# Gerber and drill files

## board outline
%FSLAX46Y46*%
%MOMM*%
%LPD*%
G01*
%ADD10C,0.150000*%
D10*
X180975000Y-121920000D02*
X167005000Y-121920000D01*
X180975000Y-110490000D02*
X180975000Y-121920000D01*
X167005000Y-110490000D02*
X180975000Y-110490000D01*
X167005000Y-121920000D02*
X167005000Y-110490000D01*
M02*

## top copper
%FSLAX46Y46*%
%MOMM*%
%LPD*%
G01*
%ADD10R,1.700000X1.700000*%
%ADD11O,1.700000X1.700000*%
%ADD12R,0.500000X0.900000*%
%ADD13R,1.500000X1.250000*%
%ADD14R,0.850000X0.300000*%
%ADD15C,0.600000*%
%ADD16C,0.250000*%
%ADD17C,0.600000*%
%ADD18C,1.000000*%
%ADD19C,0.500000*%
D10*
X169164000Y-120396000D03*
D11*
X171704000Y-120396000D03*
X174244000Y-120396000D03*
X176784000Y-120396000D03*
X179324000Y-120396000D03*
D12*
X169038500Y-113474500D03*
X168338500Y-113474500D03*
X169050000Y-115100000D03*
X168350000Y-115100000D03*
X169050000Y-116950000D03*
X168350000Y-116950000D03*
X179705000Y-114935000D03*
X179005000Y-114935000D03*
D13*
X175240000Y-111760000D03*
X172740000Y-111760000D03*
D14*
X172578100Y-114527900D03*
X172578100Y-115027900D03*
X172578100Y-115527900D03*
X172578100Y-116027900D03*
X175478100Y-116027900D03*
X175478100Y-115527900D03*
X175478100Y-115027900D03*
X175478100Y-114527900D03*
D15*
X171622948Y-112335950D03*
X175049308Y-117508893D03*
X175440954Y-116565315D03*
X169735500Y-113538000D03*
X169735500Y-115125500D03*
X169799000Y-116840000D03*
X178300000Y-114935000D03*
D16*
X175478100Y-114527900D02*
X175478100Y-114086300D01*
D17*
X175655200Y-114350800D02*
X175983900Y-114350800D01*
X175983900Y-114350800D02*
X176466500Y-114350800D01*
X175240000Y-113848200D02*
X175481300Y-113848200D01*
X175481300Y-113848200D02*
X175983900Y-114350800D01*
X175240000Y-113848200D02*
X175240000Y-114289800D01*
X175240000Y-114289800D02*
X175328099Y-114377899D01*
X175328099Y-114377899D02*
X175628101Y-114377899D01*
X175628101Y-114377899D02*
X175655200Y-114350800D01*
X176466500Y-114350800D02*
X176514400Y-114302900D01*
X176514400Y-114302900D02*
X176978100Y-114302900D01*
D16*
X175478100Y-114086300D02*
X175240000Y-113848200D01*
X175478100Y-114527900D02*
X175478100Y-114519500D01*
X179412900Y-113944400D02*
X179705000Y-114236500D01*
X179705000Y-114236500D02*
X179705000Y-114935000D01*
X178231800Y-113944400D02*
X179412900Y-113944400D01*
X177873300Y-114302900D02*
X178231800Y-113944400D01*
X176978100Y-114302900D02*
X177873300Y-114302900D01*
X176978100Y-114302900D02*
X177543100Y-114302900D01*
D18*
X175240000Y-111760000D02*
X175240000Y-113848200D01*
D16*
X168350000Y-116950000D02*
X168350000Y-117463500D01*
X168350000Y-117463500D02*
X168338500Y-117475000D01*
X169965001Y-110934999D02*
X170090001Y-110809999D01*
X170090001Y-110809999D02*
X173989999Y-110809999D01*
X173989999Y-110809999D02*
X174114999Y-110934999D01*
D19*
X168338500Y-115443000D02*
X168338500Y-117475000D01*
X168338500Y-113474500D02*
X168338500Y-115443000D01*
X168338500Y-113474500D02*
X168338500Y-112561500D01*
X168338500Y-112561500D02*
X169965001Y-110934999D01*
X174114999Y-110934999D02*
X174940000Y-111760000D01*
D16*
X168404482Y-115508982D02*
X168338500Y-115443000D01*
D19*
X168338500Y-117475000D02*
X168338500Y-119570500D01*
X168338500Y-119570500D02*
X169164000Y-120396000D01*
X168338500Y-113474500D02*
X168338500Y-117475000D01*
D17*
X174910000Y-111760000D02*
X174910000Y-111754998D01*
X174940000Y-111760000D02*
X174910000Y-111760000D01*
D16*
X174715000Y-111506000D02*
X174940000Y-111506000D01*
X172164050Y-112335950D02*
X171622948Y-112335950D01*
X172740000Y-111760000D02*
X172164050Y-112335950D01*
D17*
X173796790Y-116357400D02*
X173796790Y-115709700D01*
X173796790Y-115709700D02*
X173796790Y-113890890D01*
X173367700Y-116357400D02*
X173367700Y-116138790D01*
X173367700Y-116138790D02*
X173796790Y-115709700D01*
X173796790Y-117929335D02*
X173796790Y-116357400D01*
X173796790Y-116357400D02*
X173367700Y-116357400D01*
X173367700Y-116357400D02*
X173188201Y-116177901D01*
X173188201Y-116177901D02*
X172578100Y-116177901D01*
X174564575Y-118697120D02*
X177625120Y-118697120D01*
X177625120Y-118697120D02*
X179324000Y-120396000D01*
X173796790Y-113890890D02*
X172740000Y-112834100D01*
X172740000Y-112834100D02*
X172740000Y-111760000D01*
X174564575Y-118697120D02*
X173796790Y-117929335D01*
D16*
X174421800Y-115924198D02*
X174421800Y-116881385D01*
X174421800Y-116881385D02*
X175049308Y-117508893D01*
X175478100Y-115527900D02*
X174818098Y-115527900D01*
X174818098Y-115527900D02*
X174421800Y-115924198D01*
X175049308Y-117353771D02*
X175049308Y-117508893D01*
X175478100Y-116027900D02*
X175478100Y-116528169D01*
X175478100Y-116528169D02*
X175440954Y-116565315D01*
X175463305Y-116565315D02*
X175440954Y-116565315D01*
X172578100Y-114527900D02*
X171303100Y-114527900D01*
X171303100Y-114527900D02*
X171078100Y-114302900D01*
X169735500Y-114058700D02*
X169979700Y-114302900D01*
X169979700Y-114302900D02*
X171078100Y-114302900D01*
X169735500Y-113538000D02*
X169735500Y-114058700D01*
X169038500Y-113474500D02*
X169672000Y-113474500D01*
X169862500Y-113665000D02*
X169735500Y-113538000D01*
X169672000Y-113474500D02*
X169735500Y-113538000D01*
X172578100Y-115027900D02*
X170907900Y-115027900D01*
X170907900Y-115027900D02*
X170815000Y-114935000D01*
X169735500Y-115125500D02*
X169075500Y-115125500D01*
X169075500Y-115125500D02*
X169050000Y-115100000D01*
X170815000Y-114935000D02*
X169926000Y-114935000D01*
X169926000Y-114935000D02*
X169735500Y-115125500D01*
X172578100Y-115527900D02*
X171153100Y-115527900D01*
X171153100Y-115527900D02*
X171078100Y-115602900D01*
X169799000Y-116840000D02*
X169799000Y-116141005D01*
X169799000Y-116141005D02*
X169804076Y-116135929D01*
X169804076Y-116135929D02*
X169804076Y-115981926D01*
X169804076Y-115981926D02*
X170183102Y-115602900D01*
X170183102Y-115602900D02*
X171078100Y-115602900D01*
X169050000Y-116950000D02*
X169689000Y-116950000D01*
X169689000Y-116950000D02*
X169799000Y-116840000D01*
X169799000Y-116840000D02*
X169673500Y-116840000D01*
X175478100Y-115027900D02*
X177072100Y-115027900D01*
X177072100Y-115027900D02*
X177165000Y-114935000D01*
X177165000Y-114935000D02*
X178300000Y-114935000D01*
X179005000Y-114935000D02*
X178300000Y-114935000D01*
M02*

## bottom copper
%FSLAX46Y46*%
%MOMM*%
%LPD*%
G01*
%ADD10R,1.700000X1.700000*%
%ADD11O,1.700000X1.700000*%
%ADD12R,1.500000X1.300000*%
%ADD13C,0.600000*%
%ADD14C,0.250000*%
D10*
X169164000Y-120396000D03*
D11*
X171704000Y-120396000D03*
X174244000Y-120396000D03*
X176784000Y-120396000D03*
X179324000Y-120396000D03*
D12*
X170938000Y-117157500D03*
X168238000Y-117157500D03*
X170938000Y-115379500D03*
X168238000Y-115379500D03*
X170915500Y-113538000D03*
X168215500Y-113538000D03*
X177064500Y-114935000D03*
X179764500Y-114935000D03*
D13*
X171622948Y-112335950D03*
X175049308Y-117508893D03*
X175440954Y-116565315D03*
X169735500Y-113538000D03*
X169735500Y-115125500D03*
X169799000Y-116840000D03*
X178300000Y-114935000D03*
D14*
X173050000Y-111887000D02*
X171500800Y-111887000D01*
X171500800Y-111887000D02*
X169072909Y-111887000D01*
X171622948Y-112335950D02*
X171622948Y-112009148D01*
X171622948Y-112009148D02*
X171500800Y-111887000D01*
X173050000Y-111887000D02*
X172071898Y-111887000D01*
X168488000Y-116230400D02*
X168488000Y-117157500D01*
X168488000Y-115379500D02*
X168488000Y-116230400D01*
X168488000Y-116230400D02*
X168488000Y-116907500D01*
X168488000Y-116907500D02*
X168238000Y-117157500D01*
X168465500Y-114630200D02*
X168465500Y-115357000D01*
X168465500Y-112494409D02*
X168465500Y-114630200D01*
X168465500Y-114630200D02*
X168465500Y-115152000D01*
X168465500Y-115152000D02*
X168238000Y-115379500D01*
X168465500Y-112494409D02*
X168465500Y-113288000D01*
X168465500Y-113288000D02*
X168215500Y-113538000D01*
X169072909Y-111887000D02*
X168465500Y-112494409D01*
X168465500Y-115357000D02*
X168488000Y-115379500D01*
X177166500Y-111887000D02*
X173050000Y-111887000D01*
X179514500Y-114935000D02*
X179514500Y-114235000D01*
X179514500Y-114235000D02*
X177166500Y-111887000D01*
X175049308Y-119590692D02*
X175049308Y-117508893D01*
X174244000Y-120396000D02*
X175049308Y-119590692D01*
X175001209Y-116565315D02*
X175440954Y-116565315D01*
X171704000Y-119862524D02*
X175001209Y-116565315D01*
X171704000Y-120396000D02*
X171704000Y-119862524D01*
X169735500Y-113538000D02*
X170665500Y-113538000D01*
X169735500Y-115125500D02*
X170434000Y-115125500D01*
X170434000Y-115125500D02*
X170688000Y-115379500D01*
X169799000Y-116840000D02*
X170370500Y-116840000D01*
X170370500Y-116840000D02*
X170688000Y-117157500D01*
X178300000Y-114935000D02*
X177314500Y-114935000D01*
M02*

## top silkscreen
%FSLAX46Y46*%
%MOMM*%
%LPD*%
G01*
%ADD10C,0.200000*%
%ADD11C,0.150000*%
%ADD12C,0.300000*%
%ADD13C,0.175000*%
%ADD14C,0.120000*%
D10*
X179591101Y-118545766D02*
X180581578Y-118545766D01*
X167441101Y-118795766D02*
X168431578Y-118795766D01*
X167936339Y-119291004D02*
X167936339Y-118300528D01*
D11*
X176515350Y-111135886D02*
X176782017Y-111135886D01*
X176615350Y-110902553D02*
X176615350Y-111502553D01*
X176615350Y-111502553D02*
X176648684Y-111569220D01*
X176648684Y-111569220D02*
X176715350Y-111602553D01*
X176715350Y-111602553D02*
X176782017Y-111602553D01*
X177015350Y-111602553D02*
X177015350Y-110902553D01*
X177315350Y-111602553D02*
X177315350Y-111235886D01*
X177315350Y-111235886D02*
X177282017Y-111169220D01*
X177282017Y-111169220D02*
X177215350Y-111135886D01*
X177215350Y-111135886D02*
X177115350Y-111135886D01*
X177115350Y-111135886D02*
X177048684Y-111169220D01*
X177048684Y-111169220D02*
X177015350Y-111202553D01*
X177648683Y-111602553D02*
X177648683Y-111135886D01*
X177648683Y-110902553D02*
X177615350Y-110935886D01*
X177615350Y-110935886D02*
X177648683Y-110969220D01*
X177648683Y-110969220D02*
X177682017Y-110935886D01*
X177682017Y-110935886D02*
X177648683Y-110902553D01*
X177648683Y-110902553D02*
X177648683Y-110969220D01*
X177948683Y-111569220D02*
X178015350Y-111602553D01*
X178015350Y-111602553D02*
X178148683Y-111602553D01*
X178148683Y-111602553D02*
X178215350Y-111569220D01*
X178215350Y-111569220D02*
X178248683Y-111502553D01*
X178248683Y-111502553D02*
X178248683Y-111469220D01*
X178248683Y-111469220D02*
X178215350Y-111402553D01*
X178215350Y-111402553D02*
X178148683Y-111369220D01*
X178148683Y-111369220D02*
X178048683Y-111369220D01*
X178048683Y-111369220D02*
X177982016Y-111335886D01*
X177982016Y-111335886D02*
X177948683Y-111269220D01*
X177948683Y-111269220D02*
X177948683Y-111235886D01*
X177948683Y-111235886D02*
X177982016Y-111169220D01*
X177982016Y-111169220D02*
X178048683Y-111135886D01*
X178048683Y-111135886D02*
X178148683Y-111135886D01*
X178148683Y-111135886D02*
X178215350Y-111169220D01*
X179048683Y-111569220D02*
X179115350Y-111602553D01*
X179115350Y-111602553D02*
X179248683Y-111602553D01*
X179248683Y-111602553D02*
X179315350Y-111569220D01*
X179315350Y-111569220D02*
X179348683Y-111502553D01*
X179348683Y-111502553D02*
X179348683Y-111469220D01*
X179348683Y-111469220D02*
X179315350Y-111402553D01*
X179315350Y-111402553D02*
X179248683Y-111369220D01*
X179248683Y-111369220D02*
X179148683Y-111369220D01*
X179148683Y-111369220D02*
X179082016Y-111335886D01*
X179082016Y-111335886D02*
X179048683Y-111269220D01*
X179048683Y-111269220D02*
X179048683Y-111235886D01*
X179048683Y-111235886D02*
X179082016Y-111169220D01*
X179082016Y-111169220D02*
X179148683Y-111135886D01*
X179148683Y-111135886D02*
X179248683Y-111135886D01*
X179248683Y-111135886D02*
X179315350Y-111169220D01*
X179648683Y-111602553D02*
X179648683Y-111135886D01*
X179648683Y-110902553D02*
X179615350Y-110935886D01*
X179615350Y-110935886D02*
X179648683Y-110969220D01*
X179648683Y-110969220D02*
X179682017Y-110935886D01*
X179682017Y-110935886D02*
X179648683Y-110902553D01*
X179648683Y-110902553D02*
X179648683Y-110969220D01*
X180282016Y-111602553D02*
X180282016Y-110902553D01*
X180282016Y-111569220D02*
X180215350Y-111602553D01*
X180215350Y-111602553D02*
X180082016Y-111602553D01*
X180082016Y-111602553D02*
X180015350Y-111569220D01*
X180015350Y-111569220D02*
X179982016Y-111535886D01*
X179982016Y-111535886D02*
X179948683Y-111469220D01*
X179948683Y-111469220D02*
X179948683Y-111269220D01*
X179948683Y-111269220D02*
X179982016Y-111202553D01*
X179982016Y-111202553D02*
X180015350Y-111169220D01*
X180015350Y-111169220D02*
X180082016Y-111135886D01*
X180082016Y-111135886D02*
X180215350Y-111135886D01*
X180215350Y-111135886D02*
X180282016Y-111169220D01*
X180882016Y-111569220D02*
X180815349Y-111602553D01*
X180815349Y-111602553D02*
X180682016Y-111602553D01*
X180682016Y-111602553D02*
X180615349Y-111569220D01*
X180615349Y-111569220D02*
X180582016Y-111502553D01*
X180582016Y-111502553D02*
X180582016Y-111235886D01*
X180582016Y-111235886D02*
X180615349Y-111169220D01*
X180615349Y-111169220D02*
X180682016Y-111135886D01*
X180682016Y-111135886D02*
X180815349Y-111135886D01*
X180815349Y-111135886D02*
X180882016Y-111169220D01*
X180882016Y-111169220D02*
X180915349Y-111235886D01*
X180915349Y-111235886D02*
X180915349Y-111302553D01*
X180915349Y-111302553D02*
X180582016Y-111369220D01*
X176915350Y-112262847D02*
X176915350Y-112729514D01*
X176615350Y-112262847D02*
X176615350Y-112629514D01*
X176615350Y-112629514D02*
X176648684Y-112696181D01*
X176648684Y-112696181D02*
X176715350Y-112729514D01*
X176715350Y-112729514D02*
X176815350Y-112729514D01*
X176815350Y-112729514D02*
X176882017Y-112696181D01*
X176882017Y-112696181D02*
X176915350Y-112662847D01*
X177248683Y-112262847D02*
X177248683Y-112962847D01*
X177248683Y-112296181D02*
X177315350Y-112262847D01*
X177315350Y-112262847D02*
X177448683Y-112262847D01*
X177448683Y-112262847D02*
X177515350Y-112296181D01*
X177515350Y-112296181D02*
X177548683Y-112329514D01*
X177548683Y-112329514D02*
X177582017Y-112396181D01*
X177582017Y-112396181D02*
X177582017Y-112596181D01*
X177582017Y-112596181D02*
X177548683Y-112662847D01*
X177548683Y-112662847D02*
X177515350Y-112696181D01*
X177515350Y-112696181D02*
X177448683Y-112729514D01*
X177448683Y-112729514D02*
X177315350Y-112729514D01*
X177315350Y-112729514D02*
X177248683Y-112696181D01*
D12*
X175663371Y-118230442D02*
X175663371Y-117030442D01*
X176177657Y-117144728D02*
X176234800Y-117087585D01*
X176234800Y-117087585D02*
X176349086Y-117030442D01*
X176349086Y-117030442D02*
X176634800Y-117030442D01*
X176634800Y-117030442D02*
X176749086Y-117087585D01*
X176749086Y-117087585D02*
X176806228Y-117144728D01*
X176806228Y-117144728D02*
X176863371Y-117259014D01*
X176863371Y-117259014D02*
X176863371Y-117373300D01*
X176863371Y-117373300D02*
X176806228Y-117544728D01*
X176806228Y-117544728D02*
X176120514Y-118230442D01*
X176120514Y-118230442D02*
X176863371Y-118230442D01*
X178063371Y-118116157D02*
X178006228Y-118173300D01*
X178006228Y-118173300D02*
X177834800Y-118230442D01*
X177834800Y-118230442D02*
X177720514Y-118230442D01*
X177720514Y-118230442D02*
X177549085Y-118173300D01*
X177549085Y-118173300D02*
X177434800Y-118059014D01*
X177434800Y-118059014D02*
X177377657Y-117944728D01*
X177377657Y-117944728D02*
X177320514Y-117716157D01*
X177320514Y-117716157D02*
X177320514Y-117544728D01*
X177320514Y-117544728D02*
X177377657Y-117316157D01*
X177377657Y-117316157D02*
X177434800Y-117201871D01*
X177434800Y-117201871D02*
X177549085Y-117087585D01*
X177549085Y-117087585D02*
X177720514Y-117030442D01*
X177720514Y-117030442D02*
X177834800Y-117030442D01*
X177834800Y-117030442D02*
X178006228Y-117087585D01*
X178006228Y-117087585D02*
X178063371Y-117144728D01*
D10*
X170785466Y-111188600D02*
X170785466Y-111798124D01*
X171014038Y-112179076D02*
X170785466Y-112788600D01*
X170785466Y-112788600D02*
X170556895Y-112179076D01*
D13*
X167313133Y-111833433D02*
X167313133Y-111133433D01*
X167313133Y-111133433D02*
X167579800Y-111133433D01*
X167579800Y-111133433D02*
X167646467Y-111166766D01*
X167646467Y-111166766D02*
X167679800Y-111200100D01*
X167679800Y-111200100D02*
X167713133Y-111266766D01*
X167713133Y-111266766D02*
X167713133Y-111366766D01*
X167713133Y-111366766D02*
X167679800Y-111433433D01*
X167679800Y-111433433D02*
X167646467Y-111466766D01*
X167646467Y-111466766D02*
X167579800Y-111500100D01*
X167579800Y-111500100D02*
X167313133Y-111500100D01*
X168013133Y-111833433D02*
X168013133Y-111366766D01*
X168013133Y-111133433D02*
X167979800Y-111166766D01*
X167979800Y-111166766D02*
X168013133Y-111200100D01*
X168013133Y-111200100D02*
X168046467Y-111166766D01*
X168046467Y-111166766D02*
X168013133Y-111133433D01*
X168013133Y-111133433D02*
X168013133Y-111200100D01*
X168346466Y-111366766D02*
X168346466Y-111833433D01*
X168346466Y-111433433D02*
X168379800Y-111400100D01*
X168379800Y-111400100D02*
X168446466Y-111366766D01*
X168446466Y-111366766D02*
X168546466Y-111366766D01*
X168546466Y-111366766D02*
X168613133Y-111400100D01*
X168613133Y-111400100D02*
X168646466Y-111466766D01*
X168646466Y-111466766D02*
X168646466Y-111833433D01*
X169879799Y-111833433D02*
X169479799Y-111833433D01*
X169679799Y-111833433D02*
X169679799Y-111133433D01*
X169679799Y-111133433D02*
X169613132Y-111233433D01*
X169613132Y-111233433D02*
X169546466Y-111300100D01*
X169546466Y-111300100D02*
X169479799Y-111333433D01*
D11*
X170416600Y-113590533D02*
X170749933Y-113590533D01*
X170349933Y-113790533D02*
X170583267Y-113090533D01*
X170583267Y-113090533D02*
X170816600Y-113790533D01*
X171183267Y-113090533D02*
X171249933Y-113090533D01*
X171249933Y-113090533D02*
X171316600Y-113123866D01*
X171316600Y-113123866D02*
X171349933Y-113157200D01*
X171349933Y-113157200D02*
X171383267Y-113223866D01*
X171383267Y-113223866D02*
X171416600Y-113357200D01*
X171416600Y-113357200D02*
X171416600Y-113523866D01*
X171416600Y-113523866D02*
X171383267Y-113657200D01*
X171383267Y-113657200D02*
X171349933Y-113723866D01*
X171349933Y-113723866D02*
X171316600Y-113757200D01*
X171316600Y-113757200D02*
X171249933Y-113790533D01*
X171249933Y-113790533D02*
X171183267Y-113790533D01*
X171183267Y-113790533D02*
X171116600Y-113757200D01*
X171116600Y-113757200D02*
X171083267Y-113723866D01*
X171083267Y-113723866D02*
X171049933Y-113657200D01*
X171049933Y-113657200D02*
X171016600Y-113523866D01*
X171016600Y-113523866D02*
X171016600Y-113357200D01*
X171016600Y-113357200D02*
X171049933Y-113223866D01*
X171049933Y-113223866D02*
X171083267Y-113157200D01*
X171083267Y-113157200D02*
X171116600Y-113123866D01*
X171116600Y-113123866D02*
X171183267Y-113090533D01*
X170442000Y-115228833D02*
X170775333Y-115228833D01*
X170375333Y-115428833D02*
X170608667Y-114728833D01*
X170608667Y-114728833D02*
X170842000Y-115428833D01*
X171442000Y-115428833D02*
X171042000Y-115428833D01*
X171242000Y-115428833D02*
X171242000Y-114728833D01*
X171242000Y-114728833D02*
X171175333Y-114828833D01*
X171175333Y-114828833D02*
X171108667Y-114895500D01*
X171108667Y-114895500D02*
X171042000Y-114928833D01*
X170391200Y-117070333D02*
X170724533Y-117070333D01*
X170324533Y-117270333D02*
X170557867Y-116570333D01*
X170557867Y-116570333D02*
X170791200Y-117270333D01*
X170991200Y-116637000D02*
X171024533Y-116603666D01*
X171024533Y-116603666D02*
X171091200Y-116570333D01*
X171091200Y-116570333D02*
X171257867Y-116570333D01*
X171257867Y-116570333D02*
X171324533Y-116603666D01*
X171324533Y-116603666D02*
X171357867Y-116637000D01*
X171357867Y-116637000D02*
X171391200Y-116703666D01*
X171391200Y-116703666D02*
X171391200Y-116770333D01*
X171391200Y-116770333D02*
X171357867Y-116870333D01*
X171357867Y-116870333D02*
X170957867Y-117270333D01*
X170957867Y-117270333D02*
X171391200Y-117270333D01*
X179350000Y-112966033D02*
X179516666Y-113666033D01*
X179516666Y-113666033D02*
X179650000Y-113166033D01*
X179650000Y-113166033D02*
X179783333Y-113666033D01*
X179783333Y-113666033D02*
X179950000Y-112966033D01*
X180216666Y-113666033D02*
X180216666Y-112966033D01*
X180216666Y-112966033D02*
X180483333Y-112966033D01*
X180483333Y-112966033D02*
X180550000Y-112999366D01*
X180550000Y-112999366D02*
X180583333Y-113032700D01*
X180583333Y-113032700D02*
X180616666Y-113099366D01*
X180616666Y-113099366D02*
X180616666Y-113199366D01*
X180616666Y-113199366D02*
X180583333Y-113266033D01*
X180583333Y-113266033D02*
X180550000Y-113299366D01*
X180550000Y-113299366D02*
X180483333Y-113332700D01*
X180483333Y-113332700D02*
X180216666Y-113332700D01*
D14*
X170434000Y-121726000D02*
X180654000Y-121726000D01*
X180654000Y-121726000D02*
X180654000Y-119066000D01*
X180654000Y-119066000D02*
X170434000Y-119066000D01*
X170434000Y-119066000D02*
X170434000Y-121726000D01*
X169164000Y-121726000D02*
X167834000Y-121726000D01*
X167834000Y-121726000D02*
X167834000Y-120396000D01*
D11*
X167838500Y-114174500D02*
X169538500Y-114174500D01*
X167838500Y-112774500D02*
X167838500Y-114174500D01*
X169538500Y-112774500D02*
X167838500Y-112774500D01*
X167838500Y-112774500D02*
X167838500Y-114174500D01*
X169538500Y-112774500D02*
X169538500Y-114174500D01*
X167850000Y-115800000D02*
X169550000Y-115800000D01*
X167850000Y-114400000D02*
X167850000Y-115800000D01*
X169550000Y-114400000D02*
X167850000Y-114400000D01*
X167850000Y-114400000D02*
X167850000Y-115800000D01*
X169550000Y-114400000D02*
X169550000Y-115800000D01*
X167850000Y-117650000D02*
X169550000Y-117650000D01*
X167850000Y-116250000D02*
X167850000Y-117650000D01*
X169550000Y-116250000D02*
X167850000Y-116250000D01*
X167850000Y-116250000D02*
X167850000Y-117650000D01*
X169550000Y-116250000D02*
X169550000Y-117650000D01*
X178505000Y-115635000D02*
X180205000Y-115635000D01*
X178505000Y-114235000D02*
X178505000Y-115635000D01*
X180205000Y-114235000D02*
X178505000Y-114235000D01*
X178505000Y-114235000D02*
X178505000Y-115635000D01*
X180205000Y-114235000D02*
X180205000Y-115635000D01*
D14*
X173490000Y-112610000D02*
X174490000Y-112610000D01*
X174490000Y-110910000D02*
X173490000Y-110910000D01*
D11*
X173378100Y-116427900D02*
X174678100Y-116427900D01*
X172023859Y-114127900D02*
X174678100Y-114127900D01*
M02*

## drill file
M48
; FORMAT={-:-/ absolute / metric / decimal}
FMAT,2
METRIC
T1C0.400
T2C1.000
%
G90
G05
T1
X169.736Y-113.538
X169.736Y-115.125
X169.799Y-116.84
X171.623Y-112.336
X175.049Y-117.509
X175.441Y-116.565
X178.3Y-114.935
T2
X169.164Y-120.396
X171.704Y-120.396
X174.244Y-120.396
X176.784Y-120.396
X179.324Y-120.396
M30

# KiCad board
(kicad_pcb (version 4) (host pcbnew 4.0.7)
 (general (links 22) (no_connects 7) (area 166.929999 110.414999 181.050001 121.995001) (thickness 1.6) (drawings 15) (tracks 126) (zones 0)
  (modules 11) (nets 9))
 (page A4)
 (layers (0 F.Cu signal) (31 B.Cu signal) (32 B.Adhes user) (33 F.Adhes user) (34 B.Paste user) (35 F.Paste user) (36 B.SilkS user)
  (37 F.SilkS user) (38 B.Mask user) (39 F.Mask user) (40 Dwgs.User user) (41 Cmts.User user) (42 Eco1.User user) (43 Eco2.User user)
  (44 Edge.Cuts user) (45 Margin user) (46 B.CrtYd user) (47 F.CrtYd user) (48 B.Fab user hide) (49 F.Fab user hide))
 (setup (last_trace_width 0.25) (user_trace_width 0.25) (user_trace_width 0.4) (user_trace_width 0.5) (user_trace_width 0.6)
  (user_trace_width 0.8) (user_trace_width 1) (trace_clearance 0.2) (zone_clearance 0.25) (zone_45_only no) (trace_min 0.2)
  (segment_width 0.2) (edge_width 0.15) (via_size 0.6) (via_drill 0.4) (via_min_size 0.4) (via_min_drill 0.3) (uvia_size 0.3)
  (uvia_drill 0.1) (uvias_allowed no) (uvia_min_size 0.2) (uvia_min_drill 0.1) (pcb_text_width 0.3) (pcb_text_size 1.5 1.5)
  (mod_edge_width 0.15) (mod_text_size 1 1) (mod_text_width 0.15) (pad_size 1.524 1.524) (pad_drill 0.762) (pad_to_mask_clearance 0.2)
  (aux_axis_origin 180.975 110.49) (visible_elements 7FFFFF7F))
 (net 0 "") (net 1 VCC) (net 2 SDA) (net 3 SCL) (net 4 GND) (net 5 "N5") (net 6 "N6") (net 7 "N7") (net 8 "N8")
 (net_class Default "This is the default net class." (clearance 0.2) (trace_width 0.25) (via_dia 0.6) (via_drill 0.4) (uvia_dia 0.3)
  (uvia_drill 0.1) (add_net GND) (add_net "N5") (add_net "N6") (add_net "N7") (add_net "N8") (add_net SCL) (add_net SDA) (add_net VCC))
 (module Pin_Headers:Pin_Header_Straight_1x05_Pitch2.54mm (layer F.Cu) (at 169.164 120.396 90)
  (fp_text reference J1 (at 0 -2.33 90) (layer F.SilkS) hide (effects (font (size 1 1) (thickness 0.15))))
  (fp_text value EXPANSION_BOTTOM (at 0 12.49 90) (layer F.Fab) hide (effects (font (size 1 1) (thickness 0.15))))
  (fp_line (start -1.33 1.27) (end -1.33 11.49) (layer F.SilkS) (width 0.12))
  (fp_line (start -1.33 11.49) (end 1.33 11.49) (layer F.SilkS) (width 0.12))
  (fp_line (start 1.33 11.49) (end 1.33 1.27) (layer F.SilkS) (width 0.12))
  (fp_line (start 1.33 1.27) (end -1.33 1.27) (layer F.SilkS) (width 0.12))
  (fp_line (start -1.33 0) (end -1.33 -1.33) (layer F.SilkS) (width 0.12))
  (fp_line (start -1.33 -1.33) (end 0 -1.33) (layer F.SilkS) (width 0.12))
  (pad 1 thru_hole rect (at 0 0 90) (size 1.7 1.7) (drill 1) (layers *.Cu *.Mask) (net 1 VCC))
  (pad 2 thru_hole oval (at 0 2.54 90) (size 1.7 1.7) (drill 1) (layers *.Cu *.Mask) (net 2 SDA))
  (pad 3 thru_hole oval (at 0 5.08 90) (size 1.7 1.7) (drill 1) (layers *.Cu *.Mask) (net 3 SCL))
  (pad 4 thru_hole oval (at 0 7.62 90) (size 1.7 1.7) (drill 1) (layers *.Cu *.Mask))
  (pad 5 thru_hole oval (at 0 10.16 90) (size 1.7 1.7) (drill 1) (layers *.Cu *.Mask) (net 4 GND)))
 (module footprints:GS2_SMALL (layer F.Cu) (at 168.3385 113.4745 270)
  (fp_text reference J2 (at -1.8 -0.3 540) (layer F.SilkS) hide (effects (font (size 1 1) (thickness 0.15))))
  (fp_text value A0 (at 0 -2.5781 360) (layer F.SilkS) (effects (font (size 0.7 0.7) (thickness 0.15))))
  (fp_line (start 0.7 0.5) (end 0.7 -1.2) (layer F.SilkS) (width 0.15))
  (fp_line (start -0.7 0.5) (end 0.7 0.5) (layer F.SilkS) (width 0.15))
  (fp_line (start -0.7 -1.2) (end -0.7 0.5) (layer F.SilkS) (width 0.15))
  (fp_line (start -0.7 0.5) (end 0.7 0.5) (layer F.SilkS) (width 0.15))
  (fp_line (start -0.7 -1.2) (end 0.7 -1.2) (layer F.SilkS) (width 0.15))
  (pad 1 smd rect (at 0 -0.7 270) (size 0.9 0.5) (layers F.Cu F.Paste F.Mask) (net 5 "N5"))
  (pad 2 smd rect (at 0 0 270) (size 0.9 0.5) (layers F.Cu F.Paste F.Mask) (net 1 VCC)))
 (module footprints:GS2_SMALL (layer F.Cu) (at 168.35 115.1 270)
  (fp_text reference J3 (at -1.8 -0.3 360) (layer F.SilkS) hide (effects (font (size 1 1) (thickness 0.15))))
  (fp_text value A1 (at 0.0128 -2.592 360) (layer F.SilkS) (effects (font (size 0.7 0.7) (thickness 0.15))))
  (fp_line (start 0.7 0.5) (end 0.7 -1.2) (layer F.SilkS) (width 0.15))
  (fp_line (start -0.7 0.5) (end 0.7 0.5) (layer F.SilkS) (width 0.15))
  (fp_line (start -0.7 -1.2) (end -0.7 0.5) (layer F.SilkS) (width 0.15))
  (fp_line (start -0.7 0.5) (end 0.7 0.5) (layer F.SilkS) (width 0.15))
  (fp_line (start -0.7 -1.2) (end 0.7 -1.2) (layer F.SilkS) (width 0.15))
  (pad 1 smd rect (at 0 -0.7 270) (size 0.9 0.5) (layers F.Cu F.Paste F.Mask) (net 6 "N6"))
  (pad 2 smd rect (at 0 0 270) (size 0.9 0.5) (layers F.Cu F.Paste F.Mask) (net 1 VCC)))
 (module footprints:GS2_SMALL (layer F.Cu) (at 168.35 116.95 270)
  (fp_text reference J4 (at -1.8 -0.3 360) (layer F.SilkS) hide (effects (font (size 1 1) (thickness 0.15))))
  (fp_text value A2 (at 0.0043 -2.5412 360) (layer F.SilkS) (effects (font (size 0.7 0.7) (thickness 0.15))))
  (fp_line (start 0.7 0.5) (end 0.7 -1.2) (layer F.SilkS) (width 0.15))
  (fp_line (start -0.7 0.5) (end 0.7 0.5) (layer F.SilkS) (width 0.15))
  (fp_line (start -0.7 -1.2) (end -0.7 0.5) (layer F.SilkS) (width 0.15))
  (fp_line (start -0.7 0.5) (end 0.7 0.5) (layer F.SilkS) (width 0.15))
  (fp_line (start -0.7 -1.2) (end 0.7 -1.2) (layer F.SilkS) (width 0.15))
  (pad 1 smd rect (at 0 -0.7 270) (size 0.9 0.5) (layers F.Cu F.Paste F.Mask) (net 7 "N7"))
  (pad 2 smd rect (at 0 0 270) (size 0.9 0.5) (layers F.Cu F.Paste F.Mask) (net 1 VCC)))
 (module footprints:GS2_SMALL (layer F.Cu) (at 179.005 114.935 270)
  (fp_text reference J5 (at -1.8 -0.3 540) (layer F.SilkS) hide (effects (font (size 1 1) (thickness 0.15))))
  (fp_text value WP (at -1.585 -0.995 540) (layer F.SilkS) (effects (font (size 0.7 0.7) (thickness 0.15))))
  (fp_line (start 0.7 0.5) (end 0.7 -1.2) (layer F.SilkS) (width 0.15))
  (fp_line (start -0.7 0.5) (end 0.7 0.5) (layer F.SilkS) (width 0.15))
  (fp_line (start -0.7 -1.2) (end -0.7 0.5) (layer F.SilkS) (width 0.15))
  (fp_line (start -0.7 0.5) (end 0.7 0.5) (layer F.SilkS) (width 0.15))
  (fp_line (start -0.7 -1.2) (end 0.7 -1.2) (layer F.SilkS) (width 0.15))
  (pad 1 smd rect (at 0 -0.7 270) (size 0.9 0.5) (layers F.Cu F.Paste F.Mask) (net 1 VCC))
  (pad 2 smd rect (at 0 0 270) (size 0.9 0.5) (layers F.Cu F.Paste F.Mask) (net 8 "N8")))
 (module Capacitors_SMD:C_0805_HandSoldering (layer F.Cu) (at 173.99 111.76 180)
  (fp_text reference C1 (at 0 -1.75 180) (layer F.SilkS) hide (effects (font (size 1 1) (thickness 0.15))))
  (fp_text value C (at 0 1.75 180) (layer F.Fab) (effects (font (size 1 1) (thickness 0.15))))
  (fp_line (start 0.5 -0.85) (end -0.5 -0.85) (layer F.SilkS) (width 0.12))
  (fp_line (start -0.5 0.85) (end 0.5 0.85) (layer F.SilkS) (width 0.12))
  (pad 1 smd rect (at -1.25 0 180) (size 1.5 1.25) (layers F.Cu F.Paste F.Mask) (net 1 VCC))
  (pad 2 smd rect (at 1.25 0 180) (size 1.5 1.25) (layers F.Cu F.Paste F.Mask) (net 4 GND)))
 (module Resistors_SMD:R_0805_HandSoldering (layer B.Cu) (at 169.588 117.1575 180)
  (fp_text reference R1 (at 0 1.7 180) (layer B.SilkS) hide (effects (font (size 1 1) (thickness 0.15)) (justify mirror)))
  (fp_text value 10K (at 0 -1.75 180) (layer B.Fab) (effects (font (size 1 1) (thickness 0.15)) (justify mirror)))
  (pad 1 smd rect (at -1.35 0 180) (size 1.5 1.3) (layers B.Cu B.Paste B.Mask) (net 7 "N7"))
  (pad 2 smd rect (at 1.35 0 180) (size 1.5 1.3) (layers B.Cu B.Paste B.Mask) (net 4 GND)))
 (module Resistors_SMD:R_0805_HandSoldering (layer B.Cu) (at 169.588 115.3795 180)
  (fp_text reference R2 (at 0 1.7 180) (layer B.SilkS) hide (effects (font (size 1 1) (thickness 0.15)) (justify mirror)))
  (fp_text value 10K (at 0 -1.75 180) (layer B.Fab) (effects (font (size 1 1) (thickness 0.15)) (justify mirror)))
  (pad 1 smd rect (at -1.35 0 180) (size 1.5 1.3) (layers B.Cu B.Paste B.Mask) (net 6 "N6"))
  (pad 2 smd rect (at 1.35 0 180) (size 1.5 1.3) (layers B.Cu B.Paste B.Mask) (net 4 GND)))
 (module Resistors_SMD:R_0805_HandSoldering (layer B.Cu) (at 169.5655 113.538 180)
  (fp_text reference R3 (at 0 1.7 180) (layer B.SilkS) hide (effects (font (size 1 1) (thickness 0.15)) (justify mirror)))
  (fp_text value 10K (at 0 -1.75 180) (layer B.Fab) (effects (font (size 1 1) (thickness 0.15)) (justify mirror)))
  (pad 1 smd rect (at -1.35 0 180) (size 1.5 1.3) (layers B.Cu B.Paste B.Mask) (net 5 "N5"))
  (pad 2 smd rect (at 1.35 0 180) (size 1.5 1.3) (layers B.Cu B.Paste B.Mask) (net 4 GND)))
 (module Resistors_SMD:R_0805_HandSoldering (layer B.Cu) (at 178.4145 114.935)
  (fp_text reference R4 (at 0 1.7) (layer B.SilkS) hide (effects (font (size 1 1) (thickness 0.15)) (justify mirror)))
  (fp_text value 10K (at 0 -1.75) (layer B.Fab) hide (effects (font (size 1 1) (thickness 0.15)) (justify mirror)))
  (pad 1 smd rect (at -1.35 0) (size 1.5 1.3) (layers B.Cu B.Paste B.Mask) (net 8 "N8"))
  (pad 2 smd rect (at 1.35 0) (size 1.5 1.3) (layers B.Cu B.Paste B.Mask) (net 4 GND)))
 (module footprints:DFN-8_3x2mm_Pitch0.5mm (layer F.Cu) (at 174.0281 115.2779)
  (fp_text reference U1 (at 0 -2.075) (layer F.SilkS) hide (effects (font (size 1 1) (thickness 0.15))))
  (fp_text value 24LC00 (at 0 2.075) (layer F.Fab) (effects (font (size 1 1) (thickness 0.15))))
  (fp_line (start -0.65 1.15) (end 0.65 1.15) (layer F.SilkS) (width 0.15))
  (fp_line (start -2.004241 -1.15) (end 0.65 -1.15) (layer F.SilkS) (width 0.15))
  (pad 1 smd rect (at -1.45 -0.75) (size 0.85 0.3) (layers F.Cu F.Paste F.Mask) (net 5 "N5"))
  (pad 2 smd rect (at -1.45 -0.25) (size 0.85 0.3) (layers F.Cu F.Paste F.Mask) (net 6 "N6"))
  (pad 3 smd rect (at -1.45 0.25) (size 0.85 0.3) (layers F.Cu F.Paste F.Mask) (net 7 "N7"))
  (pad 4 smd rect (at -1.45 0.75) (size 0.85 0.3) (layers F.Cu F.Paste F.Mask) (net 4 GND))
  (pad 5 smd rect (at 1.45 0.75) (size 0.85 0.3) (layers F.Cu F.Paste F.Mask) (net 2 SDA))
  (pad 6 smd rect (at 1.45 0.25) (size 0.85 0.3) (layers F.Cu F.Paste F.Mask) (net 3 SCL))
  (pad 7 smd rect (at 1.45 -0.25) (size 0.85 0.3) (layers F.Cu F.Paste F.Mask) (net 8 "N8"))
  (pad 8 smd rect (at 1.45 -0.75) (size 0.85 0.3) (layers F.Cu F.Paste F.Mask) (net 1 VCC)))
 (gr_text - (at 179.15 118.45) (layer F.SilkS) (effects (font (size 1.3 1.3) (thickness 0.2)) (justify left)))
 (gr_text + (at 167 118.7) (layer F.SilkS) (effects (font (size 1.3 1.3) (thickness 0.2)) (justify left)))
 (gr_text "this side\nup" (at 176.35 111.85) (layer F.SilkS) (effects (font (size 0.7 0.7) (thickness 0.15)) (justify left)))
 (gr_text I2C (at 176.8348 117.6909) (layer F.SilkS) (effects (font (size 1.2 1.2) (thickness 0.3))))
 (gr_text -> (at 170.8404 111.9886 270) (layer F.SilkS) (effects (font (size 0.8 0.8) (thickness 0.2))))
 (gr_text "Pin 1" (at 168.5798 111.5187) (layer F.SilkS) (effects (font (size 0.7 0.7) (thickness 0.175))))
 (gr_line (start 180.975 121.92) (end 167.005 121.92) (layer Edge.Cuts) (width 0.15))
 (gr_line (start 180.975 110.49) (end 180.975 121.92) (layer Edge.Cuts) (width 0.15))
 (gr_line (start 167.005 110.49) (end 180.975 110.49) (layer Edge.Cuts) (width 0.15))
 (gr_line (start 167.005 121.92) (end 167.005 110.49) (layer Edge.Cuts) (width 0.15))
 (segment (start 175.4781 114.5279) (end 175.4781 114.0863) (width 0.25) (layer F.Cu) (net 1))
 (segment (start 175.6552 114.3508) (end 175.9839 114.3508) (width 0.6) (layer F.Cu) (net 1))
 (segment (start 175.9839 114.3508) (end 176.4665 114.3508) (width 0.6) (layer F.Cu) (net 1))
 (segment (start 175.24 113.8482) (end 175.4813 113.8482) (width 0.6) (layer F.Cu) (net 1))
 (segment (start 175.4813 113.8482) (end 175.9839 114.3508) (width 0.6) (layer F.Cu) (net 1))
 (segment (start 175.24 113.8482) (end 175.24 114.2898) (width 0.6) (layer F.Cu) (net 1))
 (segment (start 175.24 114.2898) (end 175.328099 114.377899) (width 0.6) (layer F.Cu) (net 1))
 (segment (start 175.328099 114.377899) (end 175.628101 114.377899) (width 0.6) (layer F.Cu) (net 1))
 (segment (start 175.628101 114.377899) (end 175.6552 114.3508) (width 0.6) (layer F.Cu) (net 1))
 (segment (start 176.4665 114.3508) (end 176.5144 114.3029) (width 0.6) (layer F.Cu) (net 1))
 (segment (start 176.5144 114.3029) (end 176.9781 114.3029) (width 0.6) (layer F.Cu) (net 1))
 (segment (start 175.4781 114.0863) (end 175.24 113.8482) (width 0.25) (layer F.Cu) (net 1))
 (segment (start 175.4781 114.5279) (end 175.4781 114.5195) (width 0.25) (layer F.Cu) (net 1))
 (segment (start 179.4129 113.9444) (end 179.705 114.2365) (width 0.25) (layer F.Cu) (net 1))
 (segment (start 179.705 114.2365) (end 179.705 114.935) (width 0.25) (layer F.Cu) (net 1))
 (segment (start 178.2318 113.9444) (end 179.4129 113.9444) (width 0.25) (layer F.Cu) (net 1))
 (segment (start 177.8733 114.3029) (end 178.2318 113.9444) (width 0.25) (layer F.Cu) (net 1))
 (segment (start 176.9781 114.3029) (end 177.8733 114.3029) (width 0.25) (layer F.Cu) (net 1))
 (segment (start 176.9781 114.3029) (end 177.5431 114.3029) (width 0.25) (layer F.Cu) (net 1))
 (segment (start 175.24 111.76) (end 175.24 113.8482) (width 1) (layer F.Cu) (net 1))
 (segment (start 168.35 116.95) (end 168.35 117.4635) (width 0.25) (layer F.Cu) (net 1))
 (segment (start 168.35 117.4635) (end 168.3385 117.475) (width 0.25) (layer F.Cu) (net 1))
 (segment (start 169.965001 110.934999) (end 170.090001 110.809999) (width 0.25) (layer F.Cu) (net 1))
 (segment (start 170.090001 110.809999) (end 173.989999 110.809999) (width 0.25) (layer F.Cu) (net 1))
 (segment (start 173.989999 110.809999) (end 174.114999 110.934999) (width 0.25) (layer F.Cu) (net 1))
 (segment (start 168.3385 115.443) (end 168.3385 117.475) (width 0.5) (layer F.Cu) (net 1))
 (segment (start 168.3385 113.4745) (end 168.3385 115.443) (width 0.5) (layer F.Cu) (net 1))
 (segment (start 168.3385 113.4745) (end 168.3385 112.5615) (width 0.5) (layer F.Cu) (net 1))
 (segment (start 168.3385 112.5615) (end 169.965001 110.934999) (width 0.5) (layer F.Cu) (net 1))
 (segment (start 174.114999 110.934999) (end 174.94 111.76) (width 0.5) (layer F.Cu) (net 1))
 (segment (start 168.404482 115.508982) (end 168.3385 115.443) (width 0.25) (layer F.Cu) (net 1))
 (segment (start 168.3385 117.475) (end 168.3385 119.5705) (width 0.5) (layer F.Cu) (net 1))
 (segment (start 168.3385 119.5705) (end 169.164 120.396) (width 0.5) (layer F.Cu) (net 1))
 (segment (start 168.3385 113.4745) (end 168.3385 117.475) (width 0.5) (layer F.Cu) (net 1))
 (segment (start 174.91 111.76) (end 174.91 111.754998) (width 0.6) (layer F.Cu) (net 1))
 (segment (start 174.94 111.76) (end 174.91 111.76) (width 0.6) (layer F.Cu) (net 1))
 (segment (start 174.715 111.506) (end 174.94 111.506) (width 0.25) (layer F.Cu) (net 1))
 (segment (start 173.05 111.887) (end 171.5008 111.887) (width 0.25) (layer B.Cu) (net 4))
 (segment (start 171.5008 111.887) (end 169.072909 111.887) (width 0.25) (layer B.Cu) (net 4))
 (segment (start 171.622948 112.33595) (end 171.622948 112.009148) (width 0.25) (layer B.Cu) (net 4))
 (segment (start 171.622948 112.009148) (end 171.5008 111.887) (width 0.25) (layer B.Cu) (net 4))
 (segment (start 173.05 111.887) (end 172.071898 111.887) (width 0.25) (layer B.Cu) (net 4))
 (segment (start 172.16405 112.33595) (end 171.622948 112.33595) (width 0.25) (layer F.Cu) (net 4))
 (segment (start 172.74 111.76) (end 172.16405 112.33595) (width 0.25) (layer F.Cu) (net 4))
 (via (at 171.622948 112.33595) (size 0.6) (drill 0.4) (layers F.Cu B.Cu) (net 4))
 (segment (start 173.79679 116.3574) (end 173.79679 115.7097) (width 0.6) (layer F.Cu) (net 4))
 (segment (start 173.79679 115.7097) (end 173.79679 113.89089) (width 0.6) (layer F.Cu) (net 4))
 (segment (start 173.3677 116.3574) (end 173.3677 116.13879) (width 0.6) (layer F.Cu) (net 4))
 (segment (start 173.3677 116.13879) (end 173.79679 115.7097) (width 0.6) (layer F.Cu) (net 4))
 (segment (start 173.79679 117.929335) (end 173.79679 116.3574) (width 0.6) (layer F.Cu) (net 4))
 (segment (start 173.79679 116.3574) (end 173.3677 116.3574) (width 0.6) (layer F.Cu) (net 4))
 (segment (start 173.3677 116.3574) (end 173.188201 116.177901) (width 0.6) (layer F.Cu) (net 4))
 (segment (start 173.188201 116.177901) (end 172.5781 116.177901) (width 0.6) (layer F.Cu) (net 4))
 (segment (start 174.564575 118.69712) (end 177.62512 118.69712) (width 0.6) (layer F.Cu) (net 4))
 (segment (start 177.62512 118.69712) (end 179.324 120.396) (width 0.6) (layer F.Cu) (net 4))
 (segment (start 173.79679 113.89089) (end 172.74 112.8341) (width 0.6) (layer F.Cu) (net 4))
 (segment (start 172.74 112.8341) (end 172.74 111.76) (width 0.6) (layer F.Cu) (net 4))
 (segment (start 174.564575 118.69712) (end 173.79679 117.929335) (width 0.6) (layer F.Cu) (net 4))
 (segment (start 168.488 116.2304) (end 168.488 117.1575) (width 0.25) (layer B.Cu) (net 4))
 (segment (start 168.488 115.3795) (end 168.488 116.2304) (width 0.25) (layer B.Cu) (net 4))
 (segment (start 168.488 116.2304) (end 168.488 116.9075) (width 0.25) (layer B.Cu) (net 4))
 (segment (start 168.488 116.9075) (end 168.238 117.1575) (width 0.25) (layer B.Cu) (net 4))
 (segment (start 168.4655 114.6302) (end 168.4655 115.357) (width 0.25) (layer B.Cu) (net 4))
 (segment (start 168.4655 112.494409) (end 168.4655 114.6302) (width 0.25) (layer B.Cu) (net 4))
 (segment (start 168.4655 114.6302) (end 168.4655 115.152) (width 0.25) (layer B.Cu) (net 4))
 (segment (start 168.4655 115.152) (end 168.238 115.3795) (width 0.25) (layer B.Cu) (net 4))
 (segment (start 168.4655 112.494409) (end 168.4655 113.288) (width 0.25) (layer B.Cu) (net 4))
 (segment (start 168.4655 113.288) (end 168.2155 113.538) (width 0.25) (layer B.Cu) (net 4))
 (segment (start 169.072909 111.887) (end 168.4655 112.494409) (width 0.25) (layer B.Cu) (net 4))
 (segment (start 168.4655 115.357) (end 168.488 115.3795) (width 0.25) (layer B.Cu) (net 4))
 (segment (start 177.1665 111.887) (end 173.05 111.887) (width 0.25) (layer B.Cu) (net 4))
 (segment (start 179.5145 114.935) (end 179.5145 114.235) (width 0.25) (layer B.Cu) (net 4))
 (segment (start 179.5145 114.235) (end 177.1665 111.887) (width 0.25) (layer B.Cu) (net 4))
 (segment (start 174.4218 115.924198) (end 174.4218 116.881385) (width 0.25) (layer F.Cu) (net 3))
 (segment (start 174.4218 116.881385) (end 175.049308 117.508893) (width 0.25) (layer F.Cu) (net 3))
 (segment (start 175.4781 115.5279) (end 174.818098 115.5279) (width 0.25) (layer F.Cu) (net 3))
 (segment (start 174.818098 115.5279) (end 174.4218 115.924198) (width 0.25) (layer F.Cu) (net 3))
 (segment (start 175.049308 117.353771) (end 175.049308 117.508893) (width 0.25) (layer F.Cu) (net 3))
 (segment (start 175.049308 119.590692) (end 175.049308 117.508893) (width 0.25) (layer B.Cu) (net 3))
 (via (at 175.049308 117.508893) (size 0.6) (drill 0.4) (layers F.Cu B.Cu) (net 3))
 (segment (start 174.244 120.396) (end 175.049308 119.590692) (width 0.25) (layer B.Cu) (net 3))
 (segment (start 175.4781 116.0279) (end 175.4781 116.528169) (width 0.25) (layer F.Cu) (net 2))
 (segment (start 175.4781 116.528169) (end 175.440954 116.565315) (width 0.25) (layer F.Cu) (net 2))
 (segment (start 175.001209 116.565315) (end 175.440954 116.565315) (width 0.25) (layer B.Cu) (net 2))
 (segment (start 171.704 119.862524) (end 175.001209 116.565315) (width 0.25) (layer B.Cu) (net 2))
 (segment (start 175.463305 116.565315) (end 175.440954 116.565315) (width 0.25) (layer F.Cu) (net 2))
 (segment (start 171.704 120.396) (end 171.704 119.862524) (width 0.25) (layer B.Cu) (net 2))
 (via (at 175.440954 116.565315) (size 0.6) (drill 0.4) (layers F.Cu B.Cu) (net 2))
 (segment (start 172.5781 114.5279) (end 171.3031 114.5279) (width 0.25) (layer F.Cu) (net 5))
 (segment (start 171.3031 114.5279) (end 171.0781 114.3029) (width 0.25) (layer F.Cu) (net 5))
 (segment (start 169.7355 114.0587) (end 169.9797 114.3029) (width 0.25) (layer F.Cu) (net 5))
 (segment (start 169.9797 114.3029) (end 171.0781 114.3029) (width 0.25) (layer F.Cu) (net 5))
 (segment (start 169.7355 113.538) (end 169.7355 114.0587) (width 0.25) (layer F.Cu) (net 5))
 (segment (start 169.0385 113.4745) (end 169.672 113.4745) (width 0.25) (layer F.Cu) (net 5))
 (segment (start 169.8625 113.665) (end 169.7355 113.538) (width 0.25) (layer F.Cu) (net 5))
 (segment (start 169.7355 113.538) (end 170.6655 113.538) (width 0.25) (layer B.Cu) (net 5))
 (segment (start 169.672 113.4745) (end 169.7355 113.538) (width 0.25) (layer F.Cu) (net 5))
 (via (at 169.7355 113.538) (size 0.6) (drill 0.4) (layers F.Cu B.Cu) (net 5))
 (segment (start 172.5781 115.0279) (end 170.9079 115.0279) (width 0.25) (layer F.Cu) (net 6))
 (segment (start 170.9079 115.0279) (end 170.815 114.935) (width 0.25) (layer F.Cu) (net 6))
 (segment (start 169.7355 115.1255) (end 169.0755 115.1255) (width 0.25) (layer F.Cu) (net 6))
 (segment (start 169.0755 115.1255) (end 169.05 115.1) (width 0.25) (layer F.Cu) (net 6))
 (segment (start 169.7355 115.1255) (end 170.434 115.1255) (width 0.25) (layer B.Cu) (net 6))
 (segment (start 170.434 115.1255) (end 170.688 115.3795) (width 0.25) (layer B.Cu) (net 6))
 (segment (start 170.815 114.935) (end 169.926 114.935) (width 0.25) (layer F.Cu) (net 6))
 (segment (start 169.926 114.935) (end 169.7355 115.1255) (width 0.25) (layer F.Cu) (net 6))
 (via (at 169.7355 115.1255) (size 0.6) (drill 0.4) (layers F.Cu B.Cu) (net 6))
 (segment (start 172.5781 115.5279) (end 171.1531 115.5279) (width 0.25) (layer F.Cu) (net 7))
 (segment (start 171.1531 115.5279) (end 171.0781 115.6029) (width 0.25) (layer F.Cu) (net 7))
 (segment (start 169.799 116.84) (end 169.799 116.141005) (width 0.25) (layer F.Cu) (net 7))
 (segment (start 169.799 116.141005) (end 169.804076 116.135929) (width 0.25) (layer F.Cu) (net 7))
 (segment (start 169.804076 116.135929) (end 169.804076 115.981926) (width 0.25) (layer F.Cu) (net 7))
 (segment (start 169.804076 115.981926) (end 170.183102 115.6029) (width 0.25) (layer F.Cu) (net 7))
 (segment (start 170.183102 115.6029) (end 171.0781 115.6029) (width 0.25) (layer F.Cu) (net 7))
 (segment (start 169.05 116.95) (end 169.689 116.95) (width 0.25) (layer F.Cu) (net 7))
 (segment (start 169.689 116.95) (end 169.799 116.84) (width 0.25) (layer F.Cu) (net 7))
 (segment (start 169.799 116.84) (end 169.6735 116.84) (width 0.25) (layer F.Cu) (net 7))
 (segment (start 169.799 116.84) (end 170.3705 116.84) (width 0.25) (layer B.Cu) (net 7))
 (segment (start 170.3705 116.84) (end 170.688 117.1575) (width 0.25) (layer B.Cu) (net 7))
 (via (at 169.799 116.84) (size 0.6) (drill 0.4) (layers F.Cu B.Cu) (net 7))
 (segment (start 175.4781 115.0279) (end 177.0721 115.0279) (width 0.25) (layer F.Cu) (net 8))
 (segment (start 177.0721 115.0279) (end 177.165 114.935) (width 0.25) (layer F.Cu) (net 8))
 (segment (start 178.3 114.935) (end 177.3145 114.935) (width 0.25) (layer B.Cu) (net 8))
 (segment (start 177.165 114.935) (end 178.3 114.935) (width 0.25) (layer F.Cu) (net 8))
 (segment (start 179.005 114.935) (end 178.3 114.935) (width 0.25) (layer F.Cu) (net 8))
 (via (at 178.3 114.935) (size 0.6) (drill 0.4) (layers F.Cu B.Cu) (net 8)))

